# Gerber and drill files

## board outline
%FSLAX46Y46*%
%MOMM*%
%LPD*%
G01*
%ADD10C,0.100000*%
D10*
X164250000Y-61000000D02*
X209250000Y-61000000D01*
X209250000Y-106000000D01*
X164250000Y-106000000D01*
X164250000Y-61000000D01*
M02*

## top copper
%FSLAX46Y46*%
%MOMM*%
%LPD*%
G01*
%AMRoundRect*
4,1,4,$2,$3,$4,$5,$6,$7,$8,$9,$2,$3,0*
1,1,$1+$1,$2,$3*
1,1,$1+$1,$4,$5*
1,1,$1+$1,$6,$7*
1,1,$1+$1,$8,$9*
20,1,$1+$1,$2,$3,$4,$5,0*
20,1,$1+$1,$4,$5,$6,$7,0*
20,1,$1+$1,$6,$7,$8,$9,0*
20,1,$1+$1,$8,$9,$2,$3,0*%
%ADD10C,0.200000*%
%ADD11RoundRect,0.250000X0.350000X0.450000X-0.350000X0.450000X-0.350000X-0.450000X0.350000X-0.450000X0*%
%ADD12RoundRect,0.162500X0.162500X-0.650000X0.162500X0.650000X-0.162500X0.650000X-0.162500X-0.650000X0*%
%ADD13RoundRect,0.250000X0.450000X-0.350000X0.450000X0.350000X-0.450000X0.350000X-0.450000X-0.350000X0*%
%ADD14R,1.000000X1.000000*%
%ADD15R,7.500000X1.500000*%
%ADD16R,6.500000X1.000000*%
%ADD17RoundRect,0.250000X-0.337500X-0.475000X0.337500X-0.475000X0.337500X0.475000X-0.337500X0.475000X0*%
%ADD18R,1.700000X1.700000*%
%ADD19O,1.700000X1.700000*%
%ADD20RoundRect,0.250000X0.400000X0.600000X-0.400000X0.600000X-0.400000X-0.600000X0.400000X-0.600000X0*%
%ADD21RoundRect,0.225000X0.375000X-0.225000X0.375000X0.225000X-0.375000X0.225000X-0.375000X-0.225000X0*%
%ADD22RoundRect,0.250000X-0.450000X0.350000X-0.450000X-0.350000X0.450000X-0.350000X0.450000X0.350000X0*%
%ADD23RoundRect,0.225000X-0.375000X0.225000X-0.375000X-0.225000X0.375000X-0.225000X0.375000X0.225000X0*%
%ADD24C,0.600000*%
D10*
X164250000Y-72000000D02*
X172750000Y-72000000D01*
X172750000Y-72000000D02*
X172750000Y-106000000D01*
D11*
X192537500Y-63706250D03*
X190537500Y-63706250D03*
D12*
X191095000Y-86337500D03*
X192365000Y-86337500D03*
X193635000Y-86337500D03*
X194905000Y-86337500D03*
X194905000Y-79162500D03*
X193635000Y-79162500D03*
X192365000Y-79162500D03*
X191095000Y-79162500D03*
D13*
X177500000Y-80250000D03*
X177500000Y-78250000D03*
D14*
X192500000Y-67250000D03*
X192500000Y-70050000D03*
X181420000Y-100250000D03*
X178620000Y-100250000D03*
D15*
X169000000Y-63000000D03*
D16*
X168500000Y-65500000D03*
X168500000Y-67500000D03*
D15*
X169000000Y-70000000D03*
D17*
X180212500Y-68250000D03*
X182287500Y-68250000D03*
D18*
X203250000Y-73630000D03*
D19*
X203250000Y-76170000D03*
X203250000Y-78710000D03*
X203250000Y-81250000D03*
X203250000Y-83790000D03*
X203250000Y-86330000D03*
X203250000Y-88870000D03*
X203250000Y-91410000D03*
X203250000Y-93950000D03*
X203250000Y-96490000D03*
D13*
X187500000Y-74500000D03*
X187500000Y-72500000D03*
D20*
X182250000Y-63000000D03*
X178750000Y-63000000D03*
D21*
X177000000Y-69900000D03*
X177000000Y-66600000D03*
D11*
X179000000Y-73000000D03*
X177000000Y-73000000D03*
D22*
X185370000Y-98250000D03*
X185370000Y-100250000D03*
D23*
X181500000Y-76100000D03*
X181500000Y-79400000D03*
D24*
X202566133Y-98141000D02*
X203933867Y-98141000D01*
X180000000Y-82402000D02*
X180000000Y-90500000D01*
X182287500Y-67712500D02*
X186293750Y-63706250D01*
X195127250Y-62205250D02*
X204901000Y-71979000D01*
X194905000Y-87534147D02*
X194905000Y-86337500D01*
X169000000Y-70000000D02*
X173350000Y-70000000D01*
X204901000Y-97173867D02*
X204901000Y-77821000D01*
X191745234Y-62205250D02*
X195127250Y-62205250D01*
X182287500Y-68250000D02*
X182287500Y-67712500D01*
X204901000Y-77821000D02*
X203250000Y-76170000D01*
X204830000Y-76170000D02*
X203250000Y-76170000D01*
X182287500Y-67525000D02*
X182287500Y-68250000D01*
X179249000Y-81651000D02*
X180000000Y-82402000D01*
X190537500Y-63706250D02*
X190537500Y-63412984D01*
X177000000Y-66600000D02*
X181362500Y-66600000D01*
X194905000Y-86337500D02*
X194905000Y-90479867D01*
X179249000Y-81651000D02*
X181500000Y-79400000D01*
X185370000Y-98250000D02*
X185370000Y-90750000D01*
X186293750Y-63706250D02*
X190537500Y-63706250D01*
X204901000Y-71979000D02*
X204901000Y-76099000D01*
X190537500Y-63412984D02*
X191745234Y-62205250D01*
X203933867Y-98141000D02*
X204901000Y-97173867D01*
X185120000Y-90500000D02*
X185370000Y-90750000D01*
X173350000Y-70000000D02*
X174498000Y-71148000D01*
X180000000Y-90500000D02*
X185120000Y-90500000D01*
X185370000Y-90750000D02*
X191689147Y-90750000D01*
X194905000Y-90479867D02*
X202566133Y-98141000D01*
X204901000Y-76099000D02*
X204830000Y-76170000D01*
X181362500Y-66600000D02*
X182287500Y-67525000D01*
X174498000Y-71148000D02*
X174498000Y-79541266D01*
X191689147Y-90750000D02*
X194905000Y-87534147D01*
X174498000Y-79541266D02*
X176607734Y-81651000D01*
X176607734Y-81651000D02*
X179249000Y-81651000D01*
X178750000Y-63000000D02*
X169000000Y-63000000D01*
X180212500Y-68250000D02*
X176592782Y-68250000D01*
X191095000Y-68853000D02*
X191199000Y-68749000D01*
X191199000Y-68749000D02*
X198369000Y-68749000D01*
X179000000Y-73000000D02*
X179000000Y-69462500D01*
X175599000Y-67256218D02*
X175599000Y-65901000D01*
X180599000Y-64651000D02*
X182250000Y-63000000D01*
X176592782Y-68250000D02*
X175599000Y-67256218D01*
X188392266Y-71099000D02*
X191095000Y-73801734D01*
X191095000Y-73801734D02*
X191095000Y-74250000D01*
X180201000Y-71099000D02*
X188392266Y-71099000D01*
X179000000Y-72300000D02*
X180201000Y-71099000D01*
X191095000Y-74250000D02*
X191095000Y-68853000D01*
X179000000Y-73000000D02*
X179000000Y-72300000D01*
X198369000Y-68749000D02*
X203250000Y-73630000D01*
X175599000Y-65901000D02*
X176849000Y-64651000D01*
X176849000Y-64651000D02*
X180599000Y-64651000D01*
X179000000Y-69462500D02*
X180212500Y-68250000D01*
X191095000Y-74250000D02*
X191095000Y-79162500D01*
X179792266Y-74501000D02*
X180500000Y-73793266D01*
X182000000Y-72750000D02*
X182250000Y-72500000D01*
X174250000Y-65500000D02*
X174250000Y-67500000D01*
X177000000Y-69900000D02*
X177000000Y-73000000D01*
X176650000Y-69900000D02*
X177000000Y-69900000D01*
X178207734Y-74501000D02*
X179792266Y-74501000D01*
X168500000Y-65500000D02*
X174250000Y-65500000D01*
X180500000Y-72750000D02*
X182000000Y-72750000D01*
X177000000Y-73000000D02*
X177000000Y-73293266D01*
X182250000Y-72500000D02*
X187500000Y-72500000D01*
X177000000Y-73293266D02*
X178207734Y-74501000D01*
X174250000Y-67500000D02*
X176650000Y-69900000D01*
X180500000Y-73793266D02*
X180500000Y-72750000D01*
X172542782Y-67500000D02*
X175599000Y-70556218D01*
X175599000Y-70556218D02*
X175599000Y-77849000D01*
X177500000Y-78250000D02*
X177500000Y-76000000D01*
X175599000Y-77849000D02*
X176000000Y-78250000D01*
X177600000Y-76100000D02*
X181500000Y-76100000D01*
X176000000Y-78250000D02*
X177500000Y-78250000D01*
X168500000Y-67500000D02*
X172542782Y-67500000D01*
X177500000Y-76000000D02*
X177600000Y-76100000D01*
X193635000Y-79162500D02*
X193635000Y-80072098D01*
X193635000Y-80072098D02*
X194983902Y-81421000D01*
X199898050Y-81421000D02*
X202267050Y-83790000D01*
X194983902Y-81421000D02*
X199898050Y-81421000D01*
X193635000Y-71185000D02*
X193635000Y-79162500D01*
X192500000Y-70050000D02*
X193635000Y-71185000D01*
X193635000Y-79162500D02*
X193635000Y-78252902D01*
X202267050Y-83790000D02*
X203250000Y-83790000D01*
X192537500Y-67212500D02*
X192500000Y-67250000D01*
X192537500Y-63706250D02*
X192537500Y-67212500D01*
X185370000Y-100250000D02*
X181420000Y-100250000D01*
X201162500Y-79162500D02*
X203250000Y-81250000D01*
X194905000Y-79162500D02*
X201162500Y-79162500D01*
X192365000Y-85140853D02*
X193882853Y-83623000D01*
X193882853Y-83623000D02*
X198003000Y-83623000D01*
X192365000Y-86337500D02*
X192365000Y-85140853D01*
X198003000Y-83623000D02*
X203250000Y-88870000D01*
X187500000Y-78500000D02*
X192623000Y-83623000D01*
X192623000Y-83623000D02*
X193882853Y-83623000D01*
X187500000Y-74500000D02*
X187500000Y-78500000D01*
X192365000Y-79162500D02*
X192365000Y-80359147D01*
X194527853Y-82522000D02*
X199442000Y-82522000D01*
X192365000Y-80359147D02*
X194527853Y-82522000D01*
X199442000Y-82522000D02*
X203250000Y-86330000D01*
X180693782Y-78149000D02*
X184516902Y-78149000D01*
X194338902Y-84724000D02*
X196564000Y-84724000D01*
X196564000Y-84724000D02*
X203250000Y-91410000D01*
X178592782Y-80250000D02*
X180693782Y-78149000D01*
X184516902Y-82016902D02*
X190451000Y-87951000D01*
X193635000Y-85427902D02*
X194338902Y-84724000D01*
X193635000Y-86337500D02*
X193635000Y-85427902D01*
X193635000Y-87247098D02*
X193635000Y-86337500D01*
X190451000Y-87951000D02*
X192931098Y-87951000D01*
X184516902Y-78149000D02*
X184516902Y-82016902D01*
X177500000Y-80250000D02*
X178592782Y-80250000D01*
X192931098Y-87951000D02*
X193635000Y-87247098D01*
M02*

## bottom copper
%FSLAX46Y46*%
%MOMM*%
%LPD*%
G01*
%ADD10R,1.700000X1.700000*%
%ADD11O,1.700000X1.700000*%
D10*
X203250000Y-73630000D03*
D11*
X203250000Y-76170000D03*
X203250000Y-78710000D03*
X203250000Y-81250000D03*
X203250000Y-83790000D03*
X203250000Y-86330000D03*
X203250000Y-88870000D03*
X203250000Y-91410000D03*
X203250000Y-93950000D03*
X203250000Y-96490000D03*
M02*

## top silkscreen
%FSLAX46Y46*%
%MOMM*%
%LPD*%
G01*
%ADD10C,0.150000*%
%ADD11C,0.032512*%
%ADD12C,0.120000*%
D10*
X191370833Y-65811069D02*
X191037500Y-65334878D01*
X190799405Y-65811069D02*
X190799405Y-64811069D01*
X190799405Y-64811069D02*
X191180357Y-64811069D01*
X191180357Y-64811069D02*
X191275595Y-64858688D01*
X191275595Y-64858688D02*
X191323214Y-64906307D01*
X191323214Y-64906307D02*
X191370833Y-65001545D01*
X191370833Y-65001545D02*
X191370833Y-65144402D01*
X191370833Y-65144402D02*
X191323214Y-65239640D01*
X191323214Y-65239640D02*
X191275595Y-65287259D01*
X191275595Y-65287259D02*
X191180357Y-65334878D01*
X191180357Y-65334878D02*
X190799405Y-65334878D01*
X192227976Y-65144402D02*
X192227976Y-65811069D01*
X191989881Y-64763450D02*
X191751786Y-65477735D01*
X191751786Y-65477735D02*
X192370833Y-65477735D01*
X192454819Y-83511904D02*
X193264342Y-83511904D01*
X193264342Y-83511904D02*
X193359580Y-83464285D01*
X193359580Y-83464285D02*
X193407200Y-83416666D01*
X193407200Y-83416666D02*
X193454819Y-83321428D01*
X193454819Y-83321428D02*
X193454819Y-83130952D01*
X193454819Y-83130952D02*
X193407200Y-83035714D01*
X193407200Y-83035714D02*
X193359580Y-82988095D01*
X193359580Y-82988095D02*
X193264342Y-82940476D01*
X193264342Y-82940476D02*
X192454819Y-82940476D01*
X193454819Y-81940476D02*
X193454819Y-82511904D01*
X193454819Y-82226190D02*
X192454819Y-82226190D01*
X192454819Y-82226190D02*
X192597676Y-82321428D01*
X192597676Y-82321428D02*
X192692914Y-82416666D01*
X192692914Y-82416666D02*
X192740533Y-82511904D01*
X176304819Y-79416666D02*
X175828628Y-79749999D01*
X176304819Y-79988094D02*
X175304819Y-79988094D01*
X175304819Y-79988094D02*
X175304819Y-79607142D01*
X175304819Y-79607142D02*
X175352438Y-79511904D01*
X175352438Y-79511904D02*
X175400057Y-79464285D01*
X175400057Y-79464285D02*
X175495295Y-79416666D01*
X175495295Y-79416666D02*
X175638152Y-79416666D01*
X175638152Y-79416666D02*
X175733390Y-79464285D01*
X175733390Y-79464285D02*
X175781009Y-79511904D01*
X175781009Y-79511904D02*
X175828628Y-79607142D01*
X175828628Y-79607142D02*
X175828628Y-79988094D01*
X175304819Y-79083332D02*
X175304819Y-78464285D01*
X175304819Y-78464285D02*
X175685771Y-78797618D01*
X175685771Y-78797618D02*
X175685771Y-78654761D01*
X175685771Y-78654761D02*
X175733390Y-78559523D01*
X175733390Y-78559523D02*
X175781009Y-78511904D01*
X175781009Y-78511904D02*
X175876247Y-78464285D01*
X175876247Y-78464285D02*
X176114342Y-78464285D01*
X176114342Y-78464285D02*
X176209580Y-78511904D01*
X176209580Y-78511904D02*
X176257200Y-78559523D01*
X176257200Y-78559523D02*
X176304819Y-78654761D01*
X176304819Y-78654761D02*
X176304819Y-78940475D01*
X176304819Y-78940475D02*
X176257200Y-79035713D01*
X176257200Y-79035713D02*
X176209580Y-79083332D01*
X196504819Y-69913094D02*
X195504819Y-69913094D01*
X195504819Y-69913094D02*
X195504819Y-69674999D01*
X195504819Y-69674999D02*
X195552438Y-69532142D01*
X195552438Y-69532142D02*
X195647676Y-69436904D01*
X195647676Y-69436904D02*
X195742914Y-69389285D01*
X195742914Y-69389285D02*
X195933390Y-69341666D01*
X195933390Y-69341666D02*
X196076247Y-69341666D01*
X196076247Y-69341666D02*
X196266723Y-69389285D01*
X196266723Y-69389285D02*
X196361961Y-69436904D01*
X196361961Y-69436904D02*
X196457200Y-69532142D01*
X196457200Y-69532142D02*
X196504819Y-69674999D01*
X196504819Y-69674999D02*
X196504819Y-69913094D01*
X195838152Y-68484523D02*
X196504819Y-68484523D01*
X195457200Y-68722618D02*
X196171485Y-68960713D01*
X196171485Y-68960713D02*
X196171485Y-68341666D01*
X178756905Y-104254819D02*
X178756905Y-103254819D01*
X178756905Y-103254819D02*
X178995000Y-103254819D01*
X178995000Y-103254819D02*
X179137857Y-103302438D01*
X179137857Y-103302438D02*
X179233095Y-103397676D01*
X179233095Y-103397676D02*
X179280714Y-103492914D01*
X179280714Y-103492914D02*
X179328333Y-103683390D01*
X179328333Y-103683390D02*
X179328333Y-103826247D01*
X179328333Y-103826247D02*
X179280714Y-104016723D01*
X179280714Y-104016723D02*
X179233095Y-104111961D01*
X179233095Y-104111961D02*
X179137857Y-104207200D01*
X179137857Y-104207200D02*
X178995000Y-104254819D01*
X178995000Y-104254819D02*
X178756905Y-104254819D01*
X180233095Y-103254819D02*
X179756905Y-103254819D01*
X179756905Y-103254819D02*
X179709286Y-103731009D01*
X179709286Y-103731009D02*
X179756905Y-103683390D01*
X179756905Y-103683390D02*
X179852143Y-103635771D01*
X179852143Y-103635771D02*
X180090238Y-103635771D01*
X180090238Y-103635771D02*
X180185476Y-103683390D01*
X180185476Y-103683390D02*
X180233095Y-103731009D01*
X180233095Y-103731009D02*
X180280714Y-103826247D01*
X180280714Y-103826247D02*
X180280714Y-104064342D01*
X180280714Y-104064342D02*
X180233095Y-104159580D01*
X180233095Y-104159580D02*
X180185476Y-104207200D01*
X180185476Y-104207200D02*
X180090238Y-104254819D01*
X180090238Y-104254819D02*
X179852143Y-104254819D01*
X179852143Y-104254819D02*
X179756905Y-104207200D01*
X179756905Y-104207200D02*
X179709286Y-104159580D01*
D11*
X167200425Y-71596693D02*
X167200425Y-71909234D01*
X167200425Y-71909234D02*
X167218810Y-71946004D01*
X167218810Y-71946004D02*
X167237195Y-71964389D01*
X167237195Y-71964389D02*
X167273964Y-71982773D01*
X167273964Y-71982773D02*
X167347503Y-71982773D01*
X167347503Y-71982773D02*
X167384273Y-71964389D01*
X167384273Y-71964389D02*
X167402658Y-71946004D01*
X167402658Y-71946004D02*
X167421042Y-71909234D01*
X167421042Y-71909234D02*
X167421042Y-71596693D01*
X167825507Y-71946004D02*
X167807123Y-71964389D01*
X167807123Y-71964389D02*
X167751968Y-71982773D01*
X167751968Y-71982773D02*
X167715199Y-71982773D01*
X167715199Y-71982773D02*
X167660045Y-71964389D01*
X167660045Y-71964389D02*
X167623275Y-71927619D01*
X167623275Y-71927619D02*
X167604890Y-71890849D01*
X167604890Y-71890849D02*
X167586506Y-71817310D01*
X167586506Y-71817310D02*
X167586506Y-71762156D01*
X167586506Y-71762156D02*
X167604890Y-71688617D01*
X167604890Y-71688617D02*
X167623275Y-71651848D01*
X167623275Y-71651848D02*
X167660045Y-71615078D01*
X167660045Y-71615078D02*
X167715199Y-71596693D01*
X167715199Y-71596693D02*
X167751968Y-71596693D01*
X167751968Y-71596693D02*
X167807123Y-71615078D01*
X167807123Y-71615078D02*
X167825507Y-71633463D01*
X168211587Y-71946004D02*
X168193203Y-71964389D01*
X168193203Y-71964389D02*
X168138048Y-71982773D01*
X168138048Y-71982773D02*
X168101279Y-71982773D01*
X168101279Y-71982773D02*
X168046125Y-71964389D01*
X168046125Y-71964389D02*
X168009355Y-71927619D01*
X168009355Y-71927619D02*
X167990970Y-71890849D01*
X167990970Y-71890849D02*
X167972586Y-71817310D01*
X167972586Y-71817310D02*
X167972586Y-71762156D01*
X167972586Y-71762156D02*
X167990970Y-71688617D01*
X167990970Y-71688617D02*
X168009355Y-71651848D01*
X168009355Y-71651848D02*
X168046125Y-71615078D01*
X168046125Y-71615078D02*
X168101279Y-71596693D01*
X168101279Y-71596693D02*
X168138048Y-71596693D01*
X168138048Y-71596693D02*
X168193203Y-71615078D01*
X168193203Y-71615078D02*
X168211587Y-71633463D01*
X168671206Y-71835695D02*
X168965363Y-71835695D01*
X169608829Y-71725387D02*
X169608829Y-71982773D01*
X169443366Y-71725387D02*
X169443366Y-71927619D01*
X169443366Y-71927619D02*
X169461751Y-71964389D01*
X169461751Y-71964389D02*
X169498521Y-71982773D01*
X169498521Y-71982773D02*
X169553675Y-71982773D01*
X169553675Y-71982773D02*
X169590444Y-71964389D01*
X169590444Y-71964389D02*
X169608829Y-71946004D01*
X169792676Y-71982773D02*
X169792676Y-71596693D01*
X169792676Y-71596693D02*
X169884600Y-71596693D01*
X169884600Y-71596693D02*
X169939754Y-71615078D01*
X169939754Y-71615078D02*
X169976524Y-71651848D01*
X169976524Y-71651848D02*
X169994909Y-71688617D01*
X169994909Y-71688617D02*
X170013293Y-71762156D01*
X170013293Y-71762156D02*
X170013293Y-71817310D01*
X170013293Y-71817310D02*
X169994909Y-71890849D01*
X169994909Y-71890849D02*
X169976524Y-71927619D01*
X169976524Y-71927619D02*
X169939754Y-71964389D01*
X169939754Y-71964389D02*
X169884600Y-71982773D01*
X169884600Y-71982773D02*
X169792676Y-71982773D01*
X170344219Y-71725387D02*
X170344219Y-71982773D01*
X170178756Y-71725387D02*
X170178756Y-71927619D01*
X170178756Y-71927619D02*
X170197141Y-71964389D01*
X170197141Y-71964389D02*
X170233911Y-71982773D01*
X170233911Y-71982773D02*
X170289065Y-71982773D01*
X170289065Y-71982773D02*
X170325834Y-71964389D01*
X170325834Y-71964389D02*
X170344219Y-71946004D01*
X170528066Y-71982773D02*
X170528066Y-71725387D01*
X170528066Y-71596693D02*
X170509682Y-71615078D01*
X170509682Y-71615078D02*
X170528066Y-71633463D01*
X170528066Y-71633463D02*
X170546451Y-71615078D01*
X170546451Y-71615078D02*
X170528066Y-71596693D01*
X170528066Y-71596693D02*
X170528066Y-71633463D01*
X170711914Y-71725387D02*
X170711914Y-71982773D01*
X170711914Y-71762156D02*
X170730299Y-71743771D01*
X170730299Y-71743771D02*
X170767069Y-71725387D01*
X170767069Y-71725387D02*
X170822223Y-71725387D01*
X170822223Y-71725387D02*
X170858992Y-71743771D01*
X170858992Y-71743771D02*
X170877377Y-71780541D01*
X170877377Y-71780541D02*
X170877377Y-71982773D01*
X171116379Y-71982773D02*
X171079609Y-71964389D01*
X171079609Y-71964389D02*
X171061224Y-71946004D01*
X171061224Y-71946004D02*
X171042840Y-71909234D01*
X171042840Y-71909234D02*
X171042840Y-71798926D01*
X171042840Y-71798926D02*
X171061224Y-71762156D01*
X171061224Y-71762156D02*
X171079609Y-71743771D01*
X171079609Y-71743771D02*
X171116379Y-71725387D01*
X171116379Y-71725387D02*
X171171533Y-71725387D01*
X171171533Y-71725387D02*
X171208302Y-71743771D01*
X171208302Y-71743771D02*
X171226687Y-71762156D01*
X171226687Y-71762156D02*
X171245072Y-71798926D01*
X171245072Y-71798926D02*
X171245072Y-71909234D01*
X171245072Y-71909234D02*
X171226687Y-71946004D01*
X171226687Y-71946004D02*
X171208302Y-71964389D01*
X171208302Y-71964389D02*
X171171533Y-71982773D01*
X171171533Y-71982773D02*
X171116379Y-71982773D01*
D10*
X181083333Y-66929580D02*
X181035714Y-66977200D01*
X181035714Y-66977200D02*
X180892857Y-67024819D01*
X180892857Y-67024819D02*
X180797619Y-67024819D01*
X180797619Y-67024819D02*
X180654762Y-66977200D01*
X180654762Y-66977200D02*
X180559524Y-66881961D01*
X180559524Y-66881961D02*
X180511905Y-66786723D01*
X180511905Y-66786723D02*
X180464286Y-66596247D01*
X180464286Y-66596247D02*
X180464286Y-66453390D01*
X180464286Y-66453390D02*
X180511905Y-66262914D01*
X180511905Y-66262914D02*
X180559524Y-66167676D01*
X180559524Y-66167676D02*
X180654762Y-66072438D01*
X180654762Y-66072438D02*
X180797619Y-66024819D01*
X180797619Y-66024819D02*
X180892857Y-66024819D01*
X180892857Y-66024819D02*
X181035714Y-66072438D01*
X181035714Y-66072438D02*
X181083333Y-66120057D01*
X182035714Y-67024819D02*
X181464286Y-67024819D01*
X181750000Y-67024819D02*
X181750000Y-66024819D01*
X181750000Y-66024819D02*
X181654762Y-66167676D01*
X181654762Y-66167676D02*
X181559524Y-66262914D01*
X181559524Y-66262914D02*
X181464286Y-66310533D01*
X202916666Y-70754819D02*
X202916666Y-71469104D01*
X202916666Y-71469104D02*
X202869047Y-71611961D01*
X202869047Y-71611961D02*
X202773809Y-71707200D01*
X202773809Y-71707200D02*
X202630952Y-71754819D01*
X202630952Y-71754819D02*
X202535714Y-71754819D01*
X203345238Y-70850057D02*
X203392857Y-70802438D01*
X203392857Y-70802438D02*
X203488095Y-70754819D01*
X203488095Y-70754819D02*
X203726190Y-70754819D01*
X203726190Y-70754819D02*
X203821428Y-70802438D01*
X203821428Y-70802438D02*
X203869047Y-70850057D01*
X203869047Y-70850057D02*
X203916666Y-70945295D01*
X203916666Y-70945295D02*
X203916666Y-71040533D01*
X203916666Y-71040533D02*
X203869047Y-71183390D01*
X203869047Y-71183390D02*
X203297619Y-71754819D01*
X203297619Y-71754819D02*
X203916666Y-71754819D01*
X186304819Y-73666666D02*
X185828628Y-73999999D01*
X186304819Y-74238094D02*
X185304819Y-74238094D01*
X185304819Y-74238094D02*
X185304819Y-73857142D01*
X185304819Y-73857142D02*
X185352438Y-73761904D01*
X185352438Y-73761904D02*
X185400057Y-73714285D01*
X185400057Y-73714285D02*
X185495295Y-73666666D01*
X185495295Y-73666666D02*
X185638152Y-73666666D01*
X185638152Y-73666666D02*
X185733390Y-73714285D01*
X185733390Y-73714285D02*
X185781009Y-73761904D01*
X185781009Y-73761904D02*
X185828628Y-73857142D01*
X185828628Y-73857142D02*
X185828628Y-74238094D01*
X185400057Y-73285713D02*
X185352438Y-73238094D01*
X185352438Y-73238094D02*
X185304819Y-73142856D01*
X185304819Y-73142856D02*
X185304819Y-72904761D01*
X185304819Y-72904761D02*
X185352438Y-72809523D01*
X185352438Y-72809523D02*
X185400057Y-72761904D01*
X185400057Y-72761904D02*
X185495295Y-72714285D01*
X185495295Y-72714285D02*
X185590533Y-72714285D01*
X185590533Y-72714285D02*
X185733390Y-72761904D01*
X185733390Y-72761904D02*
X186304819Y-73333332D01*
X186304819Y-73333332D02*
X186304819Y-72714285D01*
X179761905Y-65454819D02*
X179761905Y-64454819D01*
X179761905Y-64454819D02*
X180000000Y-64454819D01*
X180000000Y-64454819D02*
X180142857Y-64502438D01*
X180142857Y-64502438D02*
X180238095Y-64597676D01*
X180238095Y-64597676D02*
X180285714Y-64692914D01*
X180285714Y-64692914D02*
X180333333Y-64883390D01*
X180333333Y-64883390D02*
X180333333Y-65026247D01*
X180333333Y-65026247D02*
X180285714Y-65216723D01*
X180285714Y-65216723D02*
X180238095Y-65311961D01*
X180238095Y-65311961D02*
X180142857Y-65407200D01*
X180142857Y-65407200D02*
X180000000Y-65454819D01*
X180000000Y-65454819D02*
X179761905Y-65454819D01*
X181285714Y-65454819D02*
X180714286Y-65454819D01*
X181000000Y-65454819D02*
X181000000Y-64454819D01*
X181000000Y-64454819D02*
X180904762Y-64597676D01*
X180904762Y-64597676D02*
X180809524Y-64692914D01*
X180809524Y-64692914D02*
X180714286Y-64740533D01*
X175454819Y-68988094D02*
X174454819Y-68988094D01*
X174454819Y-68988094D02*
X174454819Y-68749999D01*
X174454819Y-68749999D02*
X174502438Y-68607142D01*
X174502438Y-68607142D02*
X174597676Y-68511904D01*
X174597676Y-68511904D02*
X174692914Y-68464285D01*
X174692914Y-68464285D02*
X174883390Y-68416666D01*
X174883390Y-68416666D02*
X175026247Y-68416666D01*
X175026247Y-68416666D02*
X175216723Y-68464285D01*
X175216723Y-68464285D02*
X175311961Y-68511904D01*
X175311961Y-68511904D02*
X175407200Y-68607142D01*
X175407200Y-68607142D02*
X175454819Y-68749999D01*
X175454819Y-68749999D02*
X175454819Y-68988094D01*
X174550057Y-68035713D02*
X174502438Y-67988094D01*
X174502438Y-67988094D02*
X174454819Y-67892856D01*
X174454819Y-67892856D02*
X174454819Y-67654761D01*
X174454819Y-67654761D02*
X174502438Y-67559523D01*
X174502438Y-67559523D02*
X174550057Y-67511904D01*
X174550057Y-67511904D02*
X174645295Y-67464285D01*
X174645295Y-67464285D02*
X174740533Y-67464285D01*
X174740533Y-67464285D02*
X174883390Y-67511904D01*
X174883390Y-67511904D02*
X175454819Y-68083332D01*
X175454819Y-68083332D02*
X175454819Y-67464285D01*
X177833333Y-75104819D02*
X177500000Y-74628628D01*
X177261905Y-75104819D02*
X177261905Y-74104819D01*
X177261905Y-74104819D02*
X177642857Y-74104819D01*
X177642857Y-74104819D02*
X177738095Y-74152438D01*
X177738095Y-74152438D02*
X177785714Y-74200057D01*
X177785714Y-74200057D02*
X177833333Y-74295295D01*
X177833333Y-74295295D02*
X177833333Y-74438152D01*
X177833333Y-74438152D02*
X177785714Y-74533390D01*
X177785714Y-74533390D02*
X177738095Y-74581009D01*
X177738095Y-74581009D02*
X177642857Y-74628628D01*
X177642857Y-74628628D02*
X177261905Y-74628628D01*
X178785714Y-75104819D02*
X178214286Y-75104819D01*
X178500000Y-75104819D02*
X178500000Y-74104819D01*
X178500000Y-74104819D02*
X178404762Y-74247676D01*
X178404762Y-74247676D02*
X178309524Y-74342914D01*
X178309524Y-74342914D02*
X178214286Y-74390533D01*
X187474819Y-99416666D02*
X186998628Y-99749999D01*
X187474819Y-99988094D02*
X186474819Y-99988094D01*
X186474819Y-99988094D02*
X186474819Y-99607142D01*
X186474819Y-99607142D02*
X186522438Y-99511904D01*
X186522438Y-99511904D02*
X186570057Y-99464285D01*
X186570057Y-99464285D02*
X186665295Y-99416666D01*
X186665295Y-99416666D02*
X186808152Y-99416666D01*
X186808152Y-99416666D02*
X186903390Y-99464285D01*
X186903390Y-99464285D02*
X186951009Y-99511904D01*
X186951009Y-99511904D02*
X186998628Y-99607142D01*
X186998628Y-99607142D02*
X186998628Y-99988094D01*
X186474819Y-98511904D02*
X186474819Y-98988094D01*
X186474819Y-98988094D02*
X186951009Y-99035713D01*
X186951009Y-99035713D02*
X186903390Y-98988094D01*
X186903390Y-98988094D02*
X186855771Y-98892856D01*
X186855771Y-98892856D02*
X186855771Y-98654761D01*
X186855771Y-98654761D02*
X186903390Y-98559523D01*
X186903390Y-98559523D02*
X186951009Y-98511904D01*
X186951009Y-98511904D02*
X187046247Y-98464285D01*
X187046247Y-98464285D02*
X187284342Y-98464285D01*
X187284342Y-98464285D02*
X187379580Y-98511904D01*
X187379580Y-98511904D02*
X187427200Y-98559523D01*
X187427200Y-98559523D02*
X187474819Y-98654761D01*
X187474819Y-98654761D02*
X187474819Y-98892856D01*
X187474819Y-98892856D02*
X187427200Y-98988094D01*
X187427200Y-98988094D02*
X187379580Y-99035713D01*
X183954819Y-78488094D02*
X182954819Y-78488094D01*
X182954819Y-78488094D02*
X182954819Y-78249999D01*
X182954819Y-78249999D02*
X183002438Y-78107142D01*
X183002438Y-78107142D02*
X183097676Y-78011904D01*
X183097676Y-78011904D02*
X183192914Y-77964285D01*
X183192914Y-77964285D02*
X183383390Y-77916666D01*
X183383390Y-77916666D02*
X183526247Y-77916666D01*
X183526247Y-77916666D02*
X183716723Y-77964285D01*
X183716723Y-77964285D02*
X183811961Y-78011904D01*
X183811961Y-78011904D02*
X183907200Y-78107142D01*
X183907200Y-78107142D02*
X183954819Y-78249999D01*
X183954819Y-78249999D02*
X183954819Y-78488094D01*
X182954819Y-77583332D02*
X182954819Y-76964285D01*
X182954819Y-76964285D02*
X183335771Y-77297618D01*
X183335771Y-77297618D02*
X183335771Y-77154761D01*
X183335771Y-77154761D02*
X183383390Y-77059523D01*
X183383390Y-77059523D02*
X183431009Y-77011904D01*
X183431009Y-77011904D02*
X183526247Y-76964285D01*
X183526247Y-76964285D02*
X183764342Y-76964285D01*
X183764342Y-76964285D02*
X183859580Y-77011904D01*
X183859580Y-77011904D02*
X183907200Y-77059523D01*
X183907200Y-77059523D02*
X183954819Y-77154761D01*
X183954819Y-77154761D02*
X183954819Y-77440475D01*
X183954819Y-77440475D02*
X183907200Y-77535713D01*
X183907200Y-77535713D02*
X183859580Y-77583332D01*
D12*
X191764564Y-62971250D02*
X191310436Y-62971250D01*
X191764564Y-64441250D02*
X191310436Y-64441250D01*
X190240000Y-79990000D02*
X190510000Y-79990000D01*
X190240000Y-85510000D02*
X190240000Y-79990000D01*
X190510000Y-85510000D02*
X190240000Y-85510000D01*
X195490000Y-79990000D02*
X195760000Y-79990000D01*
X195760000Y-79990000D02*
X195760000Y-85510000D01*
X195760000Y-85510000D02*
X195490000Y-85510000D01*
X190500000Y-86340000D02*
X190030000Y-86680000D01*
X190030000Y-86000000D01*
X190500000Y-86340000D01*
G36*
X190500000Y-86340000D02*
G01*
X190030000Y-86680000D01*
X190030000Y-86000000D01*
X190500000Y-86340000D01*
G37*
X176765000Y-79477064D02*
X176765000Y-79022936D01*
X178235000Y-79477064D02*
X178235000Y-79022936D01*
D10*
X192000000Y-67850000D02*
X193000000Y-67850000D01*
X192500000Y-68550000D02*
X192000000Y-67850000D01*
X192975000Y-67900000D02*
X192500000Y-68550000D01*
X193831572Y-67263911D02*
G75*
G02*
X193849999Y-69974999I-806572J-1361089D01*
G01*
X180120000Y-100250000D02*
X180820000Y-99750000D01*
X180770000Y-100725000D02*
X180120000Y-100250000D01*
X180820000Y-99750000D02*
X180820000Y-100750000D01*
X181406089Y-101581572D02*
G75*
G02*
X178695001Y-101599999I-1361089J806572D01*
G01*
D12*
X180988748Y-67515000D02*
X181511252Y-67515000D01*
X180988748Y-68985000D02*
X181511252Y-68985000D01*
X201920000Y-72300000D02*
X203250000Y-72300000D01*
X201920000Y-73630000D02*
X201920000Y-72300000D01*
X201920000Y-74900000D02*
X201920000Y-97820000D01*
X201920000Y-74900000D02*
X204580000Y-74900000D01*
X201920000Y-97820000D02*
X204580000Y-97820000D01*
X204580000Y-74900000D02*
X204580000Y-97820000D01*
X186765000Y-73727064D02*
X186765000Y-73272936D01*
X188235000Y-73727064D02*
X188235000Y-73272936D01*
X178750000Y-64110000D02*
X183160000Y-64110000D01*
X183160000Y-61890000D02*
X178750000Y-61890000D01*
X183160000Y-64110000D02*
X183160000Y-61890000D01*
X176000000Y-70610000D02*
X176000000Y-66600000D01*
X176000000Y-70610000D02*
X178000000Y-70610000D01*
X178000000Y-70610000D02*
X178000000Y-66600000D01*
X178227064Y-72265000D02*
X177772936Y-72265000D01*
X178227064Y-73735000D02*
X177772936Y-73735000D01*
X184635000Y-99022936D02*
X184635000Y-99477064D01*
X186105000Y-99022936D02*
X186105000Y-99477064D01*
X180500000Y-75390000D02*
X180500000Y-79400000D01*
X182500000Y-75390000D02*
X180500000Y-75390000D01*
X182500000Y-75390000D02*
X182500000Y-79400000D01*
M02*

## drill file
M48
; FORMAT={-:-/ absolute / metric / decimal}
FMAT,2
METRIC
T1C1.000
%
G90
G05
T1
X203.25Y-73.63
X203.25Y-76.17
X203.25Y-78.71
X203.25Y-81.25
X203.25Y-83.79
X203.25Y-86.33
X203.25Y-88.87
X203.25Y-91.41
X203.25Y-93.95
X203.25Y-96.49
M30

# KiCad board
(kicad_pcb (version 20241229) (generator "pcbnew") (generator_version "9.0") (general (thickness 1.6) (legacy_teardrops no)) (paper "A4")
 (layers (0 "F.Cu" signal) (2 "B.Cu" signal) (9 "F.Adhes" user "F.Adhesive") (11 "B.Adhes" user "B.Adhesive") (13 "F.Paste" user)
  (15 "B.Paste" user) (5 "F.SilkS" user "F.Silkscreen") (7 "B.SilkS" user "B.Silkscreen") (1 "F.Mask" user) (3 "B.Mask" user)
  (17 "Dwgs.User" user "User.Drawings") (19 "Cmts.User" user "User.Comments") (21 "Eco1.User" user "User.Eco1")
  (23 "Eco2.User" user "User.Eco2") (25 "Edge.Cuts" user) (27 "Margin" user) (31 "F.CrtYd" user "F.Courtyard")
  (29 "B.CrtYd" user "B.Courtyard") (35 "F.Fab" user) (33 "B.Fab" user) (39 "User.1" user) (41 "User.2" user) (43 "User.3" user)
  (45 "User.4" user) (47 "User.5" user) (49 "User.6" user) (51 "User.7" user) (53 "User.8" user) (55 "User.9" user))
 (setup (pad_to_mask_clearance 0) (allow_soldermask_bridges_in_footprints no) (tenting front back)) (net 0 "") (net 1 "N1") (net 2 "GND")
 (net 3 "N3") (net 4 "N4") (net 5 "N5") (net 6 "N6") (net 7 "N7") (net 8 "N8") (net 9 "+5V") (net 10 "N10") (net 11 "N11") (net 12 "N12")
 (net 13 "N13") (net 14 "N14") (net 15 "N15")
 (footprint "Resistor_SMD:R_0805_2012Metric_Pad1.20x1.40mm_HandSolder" (layer "F.Cu") (at 191.5375 63.70625 180)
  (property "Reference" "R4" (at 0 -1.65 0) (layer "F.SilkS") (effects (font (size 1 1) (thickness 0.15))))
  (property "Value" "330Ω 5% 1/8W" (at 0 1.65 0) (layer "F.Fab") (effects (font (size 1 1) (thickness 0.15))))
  (fp_line (start -0.227064 0.735) (end 0.227064 0.735) (stroke (width 0.12) (type solid)) (layer "F.SilkS"))
  (fp_line (start -0.227064 -0.735) (end 0.227064 -0.735) (stroke (width 0.12) (type solid)) (layer "F.SilkS"))
  (pad "1" smd roundrect (at -1 0 180) (size 1.2 1.4) (layers "F.Cu" "F.Mask" "F.Paste") (roundrect_rratio 0.208333) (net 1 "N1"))
  (pad "2" smd roundrect (at 1 0 180) (size 1.2 1.4) (layers "F.Cu" "F.Mask" "F.Paste") (roundrect_rratio 0.208333) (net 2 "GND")))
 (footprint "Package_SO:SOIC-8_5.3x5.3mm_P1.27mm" (layer "F.Cu") (at 193 82.75 90)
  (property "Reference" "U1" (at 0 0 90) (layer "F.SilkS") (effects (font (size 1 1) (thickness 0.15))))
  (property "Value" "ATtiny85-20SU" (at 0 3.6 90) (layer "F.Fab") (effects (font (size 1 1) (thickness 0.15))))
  (fp_line (start 2.76 -2.76) (end 2.76 -2.49) (stroke (width 0.12) (type solid)) (layer "F.SilkS"))
  (fp_line (start -2.76 -2.76) (end 2.76 -2.76) (stroke (width 0.12) (type solid)) (layer "F.SilkS"))
  (fp_line (start -2.76 -2.49) (end -2.76 -2.76) (stroke (width 0.12) (type solid)) (layer "F.SilkS"))
  (fp_line (start 2.76 2.49) (end 2.76 2.76) (stroke (width 0.12) (type solid)) (layer "F.SilkS"))
  (fp_line (start 2.76 2.76) (end -2.76 2.76) (stroke (width 0.12) (type solid)) (layer "F.SilkS"))
  (fp_line (start -2.76 2.76) (end -2.76 2.49) (stroke (width 0.12) (type solid)) (layer "F.SilkS"))
  (fp_poly (pts (xy -3.59 -2.5) (xy -3.93 -2.97) (xy -3.25 -2.97)) (stroke (width 0.12) (type solid)) (fill yes) (layer "F.SilkS"))
  (pad "1" smd roundrect (at -3.5875 -1.905 90) (size 1.625 0.65) (layers "F.Cu" "F.Mask" "F.Paste") (roundrect_rratio 0.25) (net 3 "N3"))
  (pad "2" smd roundrect (at -3.5875 -0.635 90) (size 1.625 0.65) (layers "F.Cu" "F.Mask" "F.Paste") (roundrect_rratio 0.25) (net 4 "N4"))
  (pad "3" smd roundrect (at -3.5875 0.635 90) (size 1.625 0.65) (layers "F.Cu" "F.Mask" "F.Paste") (roundrect_rratio 0.25) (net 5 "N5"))
  (pad "4" smd roundrect (at -3.5875 1.905 90) (size 1.625 0.65) (layers "F.Cu" "F.Mask" "F.Paste") (roundrect_rratio 0.25) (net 2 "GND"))
  (pad "5" smd roundrect (at 3.5875 1.905 90) (size 1.625 0.65) (layers "F.Cu" "F.Mask" "F.Paste") (roundrect_rratio 0.25) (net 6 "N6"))
  (pad "6" smd roundrect (at 3.5875 0.635 90) (size 1.625 0.65) (layers "F.Cu" "F.Mask" "F.Paste") (roundrect_rratio 0.25) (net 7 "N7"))
  (pad "7" smd roundrect (at 3.5875 -0.635 90) (size 1.625 0.65) (layers "F.Cu" "F.Mask" "F.Paste") (roundrect_rratio 0.25) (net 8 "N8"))
  (pad "8" smd roundrect (at 3.5875 -1.905 90) (size 1.625 0.65) (layers "F.Cu" "F.Mask" "F.Paste") (roundrect_rratio 0.25) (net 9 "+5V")))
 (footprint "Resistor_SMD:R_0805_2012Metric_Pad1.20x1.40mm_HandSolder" (layer "F.Cu") (at 177.5 79.25 90)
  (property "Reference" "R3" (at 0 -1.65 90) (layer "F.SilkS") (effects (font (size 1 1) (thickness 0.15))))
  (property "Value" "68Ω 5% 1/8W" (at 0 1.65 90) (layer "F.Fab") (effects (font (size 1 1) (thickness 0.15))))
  (fp_line (start -0.227064 -0.735) (end 0.227064 -0.735) (stroke (width 0.12) (type solid)) (layer "F.SilkS"))
  (fp_line (start -0.227064 0.735) (end 0.227064 0.735) (stroke (width 0.12) (type solid)) (layer "F.SilkS"))
  (pad "1" smd roundrect (at -1 0 90) (size 1.2 1.4) (layers "F.Cu" "F.Mask" "F.Paste") (roundrect_rratio 0.208333) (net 5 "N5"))
  (pad "2" smd roundrect (at 1 0 90) (size 1.2 1.4) (layers "F.Cu" "F.Mask" "F.Paste") (roundrect_rratio 0.208333) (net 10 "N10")))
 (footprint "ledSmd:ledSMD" (layer "F.Cu") (at 192.5 69.05 -90)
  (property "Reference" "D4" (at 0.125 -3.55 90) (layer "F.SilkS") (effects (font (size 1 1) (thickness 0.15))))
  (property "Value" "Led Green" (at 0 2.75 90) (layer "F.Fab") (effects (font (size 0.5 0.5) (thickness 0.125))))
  (fp_line (start -1.2 0.5) (end -1.2 -0.5) (stroke (width 0.15) (type solid)) (layer "F.SilkS"))
  (fp_line (start -0.5 0) (end -1.2 0.5) (stroke (width 0.15) (type solid)) (layer "F.SilkS"))
  (fp_line (start -1.15 -0.475) (end -0.5 0) (stroke (width 0.15) (type solid)) (layer "F.SilkS"))
  (fp_arc (start -1.786089 -1.331572) (mid -0.435753 -2.107089) (end 0.924999 -1.349999) (stroke (width 0.15) (type solid))
   (layer "F.SilkS"))
  (pad "1" smd rect (at -1.8 0 270) (size 1 1) (layers "F.Cu" "F.Mask" "F.Paste") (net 1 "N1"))
  (pad "2" smd rect (at 1 0 270) (size 1 1) (layers "F.Cu" "F.Mask" "F.Paste") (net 7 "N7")))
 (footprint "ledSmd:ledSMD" (layer "F.Cu") (at 179.62 100.25 180)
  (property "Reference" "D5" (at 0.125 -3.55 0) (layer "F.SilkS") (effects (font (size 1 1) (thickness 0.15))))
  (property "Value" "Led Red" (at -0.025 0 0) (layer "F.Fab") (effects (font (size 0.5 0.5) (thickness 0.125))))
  (fp_line (start -0.5 0) (end -1.2 0.5) (stroke (width 0.15) (type solid)) (layer "F.SilkS"))
  (fp_line (start -1.15 -0.475) (end -0.5 0) (stroke (width 0.15) (type solid)) (layer "F.SilkS"))
  (fp_line (start -1.2 0.5) (end -1.2 -0.5) (stroke (width 0.15) (type solid)) (layer "F.SilkS"))
  (fp_arc (start -1.786089 -1.331572) (mid -0.435753 -2.107089) (end 0.924999 -1.349999) (stroke (width 0.15) (type solid))
   (layer "F.SilkS"))
  (pad "1" smd rect (at -1.8 0 180) (size 1 1) (layers "F.Cu" "F.Mask" "F.Paste") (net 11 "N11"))
  (pad "2" smd rect (at 1 0 180) (size 1 1) (layers "F.Cu" "F.Mask" "F.Paste") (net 9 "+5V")))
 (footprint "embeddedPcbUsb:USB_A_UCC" (layer "F.Cu") (at 168.8 66.5 180)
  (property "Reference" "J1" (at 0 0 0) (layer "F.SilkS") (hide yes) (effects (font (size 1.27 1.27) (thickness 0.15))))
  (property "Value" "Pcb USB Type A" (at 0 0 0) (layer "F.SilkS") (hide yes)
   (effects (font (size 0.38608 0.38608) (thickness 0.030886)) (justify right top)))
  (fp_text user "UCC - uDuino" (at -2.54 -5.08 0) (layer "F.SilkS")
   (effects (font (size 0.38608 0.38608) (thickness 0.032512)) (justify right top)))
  (pad "1" smd rect (at -0.2 3.5 180) (size 7.5 1.5) (layers "F.Cu" "F.Mask" "F.Paste") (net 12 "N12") (solder_mask_margin 0.1016))
  (pad "2" smd rect (at 0.3 1 180) (size 6.5 1) (layers "F.Cu" "F.Mask" "F.Paste") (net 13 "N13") (solder_mask_margin 0.1016))
  (pad "3" smd rect (at 0.3 -1 180) (size 6.5 1) (layers "F.Cu" "F.Mask" "F.Paste") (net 10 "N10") (solder_mask_margin 0.1016))
  (pad "4" smd rect (at -0.2 -3.5 180) (size 7.5 1.5) (layers "F.Cu" "F.Mask" "F.Paste") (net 2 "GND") (solder_mask_margin 0.1016)))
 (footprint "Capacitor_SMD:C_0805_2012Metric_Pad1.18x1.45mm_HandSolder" (layer "F.Cu") (at 181.25 68.25)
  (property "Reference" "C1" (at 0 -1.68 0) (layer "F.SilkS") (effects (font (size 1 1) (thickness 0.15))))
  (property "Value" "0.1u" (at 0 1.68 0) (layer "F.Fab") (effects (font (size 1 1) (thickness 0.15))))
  (fp_line (start -0.261252 -0.735) (end 0.261252 -0.735) (stroke (width 0.12) (type solid)) (layer "F.SilkS"))
  (fp_line (start -0.261252 0.735) (end 0.261252 0.735) (stroke (width 0.12) (type solid)) (layer "F.SilkS"))
  (pad "1" smd roundrect (at -1.0375 0) (size 1.175 1.45) (layers "F.Cu" "F.Mask" "F.Paste") (roundrect_rratio 0.212766) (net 9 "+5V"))
  (pad "2" smd roundrect (at 1.0375 0) (size 1.175 1.45) (layers "F.Cu" "F.Mask" "F.Paste") (roundrect_rratio 0.212766) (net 2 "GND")))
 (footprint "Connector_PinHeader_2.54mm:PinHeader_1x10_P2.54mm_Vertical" (layer "F.Cu") (at 203.25 73.63)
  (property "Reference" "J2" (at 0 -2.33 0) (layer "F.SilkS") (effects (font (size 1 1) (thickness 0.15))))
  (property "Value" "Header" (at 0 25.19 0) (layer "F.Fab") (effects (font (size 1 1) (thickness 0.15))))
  (fp_line (start -1.33 -1.33) (end 0 -1.33) (stroke (width 0.12) (type solid)) (layer "F.SilkS"))
  (fp_line (start -1.33 0) (end -1.33 -1.33) (stroke (width 0.12) (type solid)) (layer "F.SilkS"))
  (fp_line (start -1.33 1.27) (end -1.33 24.19) (stroke (width 0.12) (type solid)) (layer "F.SilkS"))
  (fp_line (start -1.33 1.27) (end 1.33 1.27) (stroke (width 0.12) (type solid)) (layer "F.SilkS"))
  (fp_line (start -1.33 24.19) (end 1.33 24.19) (stroke (width 0.12) (type solid)) (layer "F.SilkS"))
  (fp_line (start 1.33 1.27) (end 1.33 24.19) (stroke (width 0.12) (type solid)) (layer "F.SilkS"))
  (pad "1" thru_hole rect (at 0 0) (size 1.7 1.7) (drill 1) (layers "*.Cu" "*.Mask") (remove_unused_layers no) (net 9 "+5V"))
  (pad "2" thru_hole oval (at 0 2.54) (size 1.7 1.7) (drill 1) (layers "*.Cu" "*.Mask") (remove_unused_layers no) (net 2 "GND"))
  (pad "3" thru_hole oval (at 0 5.08) (size 1.7 1.7) (drill 1) (layers "*.Cu" "*.Mask") (remove_unused_layers no) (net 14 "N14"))
  (pad "4" thru_hole oval (at 0 7.62) (size 1.7 1.7) (drill 1) (layers "*.Cu" "*.Mask") (remove_unused_layers no) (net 6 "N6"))
  (pad "5" thru_hole oval (at 0 10.16) (size 1.7 1.7) (drill 1) (layers "*.Cu" "*.Mask") (remove_unused_layers no) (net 7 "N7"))
  (pad "6" thru_hole oval (at 0 12.7) (size 1.7 1.7) (drill 1) (layers "*.Cu" "*.Mask") (remove_unused_layers no) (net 8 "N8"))
  (pad "7" thru_hole oval (at 0 15.24) (size 1.7 1.7) (drill 1) (layers "*.Cu" "*.Mask") (remove_unused_layers no) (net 4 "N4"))
  (pad "8" thru_hole oval (at 0 17.78) (size 1.7 1.7) (drill 1) (layers "*.Cu" "*.Mask") (remove_unused_layers no) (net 5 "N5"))
  (pad "9" thru_hole oval (at 0 20.32) (size 1.7 1.7) (drill 1) (layers "*.Cu" "*.Mask") (remove_unused_layers no) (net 3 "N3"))
  (pad "10" thru_hole oval (at 0 22.86) (size 1.7 1.7) (drill 1) (layers "*.Cu" "*.Mask") (remove_unused_layers no) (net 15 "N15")))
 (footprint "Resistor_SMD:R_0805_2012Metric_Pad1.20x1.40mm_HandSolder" (layer "F.Cu") (at 187.5 73.5 90)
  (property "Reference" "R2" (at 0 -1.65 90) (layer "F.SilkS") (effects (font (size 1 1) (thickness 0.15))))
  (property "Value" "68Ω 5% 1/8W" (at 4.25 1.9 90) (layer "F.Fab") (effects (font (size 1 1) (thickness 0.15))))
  (fp_line (start -0.227064 -0.735) (end 0.227064 -0.735) (stroke (width 0.12) (type solid)) (layer "F.SilkS"))
  (fp_line (start -0.227064 0.735) (end 0.227064 0.735) (stroke (width 0.12) (type solid)) (layer "F.SilkS"))
  (pad "1" smd roundrect (at -1 0 90) (size 1.2 1.4) (layers "F.Cu" "F.Mask" "F.Paste") (roundrect_rratio 0.208333) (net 4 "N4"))
  (pad "2" smd roundrect (at 1 0 90) (size 1.2 1.4) (layers "F.Cu" "F.Mask" "F.Paste") (roundrect_rratio 0.208333) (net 13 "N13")))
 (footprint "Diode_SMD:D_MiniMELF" (layer "F.Cu") (at 180.5 63 180)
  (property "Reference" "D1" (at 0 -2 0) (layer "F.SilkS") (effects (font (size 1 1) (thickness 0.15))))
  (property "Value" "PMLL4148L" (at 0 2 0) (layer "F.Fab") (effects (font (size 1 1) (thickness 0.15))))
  (fp_line (start 1.75 -1.11) (end -2.66 -1.11) (stroke (width 0.12) (type solid)) (layer "F.SilkS"))
  (fp_line (start -2.66 1.11) (end 1.75 1.11) (stroke (width 0.12) (type solid)) (layer "F.SilkS"))
  (fp_line (start -2.66 -1.11) (end -2.66 1.11) (stroke (width 0.12) (type solid)) (layer "F.SilkS"))
  (pad "1" smd roundrect (at -1.75 0 180) (size 1.3 1.7) (layers "F.Cu" "F.Mask" "F.Paste") (roundrect_rratio 0.1923076923) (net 9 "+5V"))
  (pad "2" smd roundrect (at 1.75 0 180) (size 1.3 1.7) (layers "F.Cu" "F.Mask" "F.Paste") (roundrect_rratio 0.1923076923) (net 12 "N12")))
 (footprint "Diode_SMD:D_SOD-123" (layer "F.Cu") (at 177 68.25 90)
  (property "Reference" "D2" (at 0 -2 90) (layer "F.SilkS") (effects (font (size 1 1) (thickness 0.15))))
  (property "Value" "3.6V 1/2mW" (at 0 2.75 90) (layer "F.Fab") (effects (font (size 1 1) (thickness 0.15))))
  (fp_line (start -2.36 -1) (end 1.65 -1) (stroke (width 0.12) (type solid)) (layer "F.SilkS"))
  (fp_line (start -2.36 -1) (end -2.36 1) (stroke (width 0.12) (type solid)) (layer "F.SilkS"))
  (fp_line (start -2.36 1) (end 1.65 1) (stroke (width 0.12) (type solid)) (layer "F.SilkS"))
  (pad "1" smd roundrect (at -1.65 0 90) (size 0.9 1.2) (layers "F.Cu" "F.Mask" "F.Paste") (roundrect_rratio 0.25) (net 13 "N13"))
  (pad "2" smd roundrect (at 1.65 0 90) (size 0.9 1.2) (layers "F.Cu" "F.Mask" "F.Paste") (roundrect_rratio 0.25) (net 2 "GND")))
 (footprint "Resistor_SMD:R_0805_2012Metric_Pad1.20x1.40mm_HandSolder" (layer "F.Cu") (at 178 73 180)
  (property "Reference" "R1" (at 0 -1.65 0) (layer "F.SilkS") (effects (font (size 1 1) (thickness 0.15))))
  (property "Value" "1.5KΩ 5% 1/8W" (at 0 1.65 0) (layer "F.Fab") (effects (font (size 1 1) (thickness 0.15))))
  (fp_line (start -0.227064 0.735) (end 0.227064 0.735) (stroke (width 0.12) (type solid)) (layer "F.SilkS"))
  (fp_line (start -0.227064 -0.735) (end 0.227064 -0.735) (stroke (width 0.12) (type solid)) (layer "F.SilkS"))
  (pad "1" smd roundrect (at -1 0 180) (size 1.2 1.4) (layers "F.Cu" "F.Mask" "F.Paste") (roundrect_rratio 0.208333) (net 9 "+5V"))
  (pad "2" smd roundrect (at 1 0 180) (size 1.2 1.4) (layers "F.Cu" "F.Mask" "F.Paste") (roundrect_rratio 0.208333) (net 13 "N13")))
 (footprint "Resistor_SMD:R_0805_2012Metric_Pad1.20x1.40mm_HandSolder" (layer "F.Cu") (at 185.37 99.25 -90)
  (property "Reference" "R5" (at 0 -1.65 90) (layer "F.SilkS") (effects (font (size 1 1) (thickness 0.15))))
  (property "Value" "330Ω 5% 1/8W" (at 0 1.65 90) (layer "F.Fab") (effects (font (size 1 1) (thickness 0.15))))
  (fp_line (start -0.227064 0.735) (end 0.227064 0.735) (stroke (width 0.12) (type solid)) (layer "F.SilkS"))
  (fp_line (start -0.227064 -0.735) (end 0.227064 -0.735) (stroke (width 0.12) (type solid)) (layer "F.SilkS"))
  (pad "1" smd roundrect (at -1 0 270) (size 1.2 1.4) (layers "F.Cu" "F.Mask" "F.Paste") (roundrect_rratio 0.208333) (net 2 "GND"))
  (pad "2" smd roundrect (at 1 0 270) (size 1.2 1.4) (layers "F.Cu" "F.Mask" "F.Paste") (roundrect_rratio 0.208333) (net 11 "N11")))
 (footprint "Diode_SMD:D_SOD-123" (layer "F.Cu") (at 181.5 77.75 -90)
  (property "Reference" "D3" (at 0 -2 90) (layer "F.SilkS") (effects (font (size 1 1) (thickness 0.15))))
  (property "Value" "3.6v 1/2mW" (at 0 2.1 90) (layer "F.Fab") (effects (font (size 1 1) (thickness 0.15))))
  (fp_line (start -2.36 1) (end 1.65 1) (stroke (width 0.12) (type solid)) (layer "F.SilkS"))
  (fp_line (start -2.36 -1) (end -2.36 1) (stroke (width 0.12) (type solid)) (layer "F.SilkS"))
  (fp_line (start -2.36 -1) (end 1.65 -1) (stroke (width 0.12) (type solid)) (layer "F.SilkS"))
  (pad "1" smd roundrect (at -1.65 0 270) (size 0.9 1.2) (layers "F.Cu" "F.Mask" "F.Paste") (roundrect_rratio 0.25) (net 10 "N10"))
  (pad "2" smd roundrect (at 1.65 0 270) (size 0.9 1.2) (layers "F.Cu" "F.Mask" "F.Paste") (roundrect_rratio 0.25) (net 2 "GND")))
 (gr_line (start 164.25 72) (end 172.75 72) (stroke (width 0.2) (type default)) (layer "F.Cu"))
 (gr_line (start 172.75 72) (end 172.75 106) (stroke (width 0.2) (type default)) (layer "F.Cu"))
 (gr_rect (start 164.25 61) (end 209.25 106) (stroke (width 0.1) (type default)) (fill no) (layer "Edge.Cuts"))
 (segment (start 202.566133 98.141) (end 203.933867 98.141) (width 0.6) (layer "F.Cu") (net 2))
 (segment (start 180 82.402) (end 180 90.5) (width 0.6) (layer "F.Cu") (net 2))
 (segment (start 182.2875 67.7125) (end 186.29375 63.70625) (width 0.6) (layer "F.Cu") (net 2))
 (segment (start 195.12725 62.20525) (end 204.901 71.979) (width 0.6) (layer "F.Cu") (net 2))
 (segment (start 194.905 87.534147) (end 194.905 86.3375) (width 0.6) (layer "F.Cu") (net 2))
 (segment (start 169 70) (end 173.35 70) (width 0.6) (layer "F.Cu") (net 2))
 (segment (start 204.901 97.173867) (end 204.901 77.821) (width 0.6) (layer "F.Cu") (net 2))
 (segment (start 191.745234 62.20525) (end 195.12725 62.20525) (width 0.6) (layer "F.Cu") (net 2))
 (segment (start 182.2875 68.25) (end 182.2875 67.7125) (width 0.6) (layer "F.Cu") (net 2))
 (segment (start 204.901 77.821) (end 203.25 76.17) (width 0.6) (layer "F.Cu") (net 2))
 (segment (start 204.83 76.17) (end 203.25 76.17) (width 0.6) (layer "F.Cu") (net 2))
 (segment (start 182.2875 67.525) (end 182.2875 68.25) (width 0.6) (layer "F.Cu") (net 2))
 (segment (start 179.249 81.651) (end 180 82.402) (width 0.6) (layer "F.Cu") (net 2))
 (segment (start 190.5375 63.70625) (end 190.5375 63.412984) (width 0.6) (layer "F.Cu") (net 2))
 (segment (start 177 66.6) (end 181.3625 66.6) (width 0.6) (layer "F.Cu") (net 2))
 (segment (start 194.905 86.3375) (end 194.905 90.479867) (width 0.6) (layer "F.Cu") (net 2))
 (segment (start 179.249 81.651) (end 181.5 79.4) (width 0.6) (layer "F.Cu") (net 2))
 (segment (start 185.37 98.25) (end 185.37 90.75) (width 0.6) (layer "F.Cu") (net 2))
 (segment (start 186.29375 63.70625) (end 190.5375 63.70625) (width 0.6) (layer "F.Cu") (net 2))
 (segment (start 204.901 71.979) (end 204.901 76.099) (width 0.6) (layer "F.Cu") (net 2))
 (segment (start 190.5375 63.412984) (end 191.745234 62.20525) (width 0.6) (layer "F.Cu") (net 2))
 (segment (start 203.933867 98.141) (end 204.901 97.173867) (width 0.6) (layer "F.Cu") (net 2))
 (segment (start 185.12 90.5) (end 185.37 90.75) (width 0.6) (layer "F.Cu") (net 2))
 (segment (start 173.35 70) (end 174.498 71.148) (width 0.6) (layer "F.Cu") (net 2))
 (segment (start 180 90.5) (end 185.12 90.5) (width 0.6) (layer "F.Cu") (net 2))
 (segment (start 185.37 90.75) (end 191.689147 90.75) (width 0.6) (layer "F.Cu") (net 2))
 (segment (start 194.905 90.479867) (end 202.566133 98.141) (width 0.6) (layer "F.Cu") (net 2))
 (segment (start 204.901 76.099) (end 204.83 76.17) (width 0.6) (layer "F.Cu") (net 2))
 (segment (start 181.3625 66.6) (end 182.2875 67.525) (width 0.6) (layer "F.Cu") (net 2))
 (segment (start 174.498 71.148) (end 174.498 79.541266) (width 0.6) (layer "F.Cu") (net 2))
 (segment (start 191.689147 90.75) (end 194.905 87.534147) (width 0.6) (layer "F.Cu") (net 2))
 (segment (start 174.498 79.541266) (end 176.607734 81.651) (width 0.6) (layer "F.Cu") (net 2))
 (segment (start 176.607734 81.651) (end 179.249 81.651) (width 0.6) (layer "F.Cu") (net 2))
 (segment (start 178.75 63) (end 169 63) (width 0.6) (layer "F.Cu") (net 12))
 (segment (start 180.2125 68.25) (end 176.592782 68.25) (width 0.6) (layer "F.Cu") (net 9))
 (segment (start 191.095 68.853) (end 191.199 68.749) (width 0.6) (layer "F.Cu") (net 9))
 (segment (start 191.199 68.749) (end 198.369 68.749) (width 0.6) (layer "F.Cu") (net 9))
 (segment (start 179 73) (end 179 69.4625) (width 0.6) (layer "F.Cu") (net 9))
 (segment (start 175.599 67.256218) (end 175.599 65.901) (width 0.6) (layer "F.Cu") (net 9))
 (segment (start 180.599 64.651) (end 182.25 63) (width 0.6) (layer "F.Cu") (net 9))
 (segment (start 176.592782 68.25) (end 175.599 67.256218) (width 0.6) (layer "F.Cu") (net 9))
 (segment (start 188.392266 71.099) (end 191.095 73.801734) (width 0.6) (layer "F.Cu") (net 9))
 (segment (start 191.095 73.801734) (end 191.095 74.25) (width 0.6) (layer "F.Cu") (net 9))
 (segment (start 180.201 71.099) (end 188.392266 71.099) (width 0.6) (layer "F.Cu") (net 9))
 (segment (start 179 72.3) (end 180.201 71.099) (width 0.6) (layer "F.Cu") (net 9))
 (segment (start 191.095 74.25) (end 191.095 68.853) (width 0.6) (layer "F.Cu") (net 9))
 (segment (start 179 73) (end 179 72.3) (width 0.6) (layer "F.Cu") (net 9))
 (segment (start 198.369 68.749) (end 203.25 73.63) (width 0.6) (layer "F.Cu") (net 9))
 (segment (start 175.599 65.901) (end 176.849 64.651) (width 0.6) (layer "F.Cu") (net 9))
 (segment (start 176.849 64.651) (end 180.599 64.651) (width 0.6) (layer "F.Cu") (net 9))
 (segment (start 179 69.4625) (end 180.2125 68.25) (width 0.6) (layer "F.Cu") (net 9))
 (segment (start 191.095 74.25) (end 191.095 79.1625) (width 0.6) (layer "F.Cu") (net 9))
 (segment (start 179.792266 74.501) (end 180.5 73.793266) (width 0.6) (layer "F.Cu") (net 13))
 (segment (start 182 72.75) (end 182.25 72.5) (width 0.6) (layer "F.Cu") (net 13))
 (segment (start 174.25 65.5) (end 174.25 67.5) (width 0.6) (layer "F.Cu") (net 13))
 (segment (start 177 69.9) (end 177 73) (width 0.6) (layer "F.Cu") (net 13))
 (segment (start 176.65 69.9) (end 177 69.9) (width 0.6) (layer "F.Cu") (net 13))
 (segment (start 178.207734 74.501) (end 179.792266 74.501) (width 0.6) (layer "F.Cu") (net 13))
 (segment (start 168.5 65.5) (end 174.25 65.5) (width 0.6) (layer "F.Cu") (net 13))
 (segment (start 180.5 72.75) (end 182 72.75) (width 0.6) (layer "F.Cu") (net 13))
 (segment (start 177 73) (end 177 73.293266) (width 0.6) (layer "F.Cu") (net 13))
 (segment (start 182.25 72.5) (end 187.5 72.5) (width 0.6) (layer "F.Cu") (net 13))
 (segment (start 177 73.293266) (end 178.207734 74.501) (width 0.6) (layer "F.Cu") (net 13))
 (segment (start 174.25 67.5) (end 176.65 69.9) (width 0.6) (layer "F.Cu") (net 13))
 (segment (start 180.5 73.793266) (end 180.5 72.75) (width 0.6) (layer "F.Cu") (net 13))
 (segment (start 172.542782 67.5) (end 175.599 70.556218) (width 0.6) (layer "F.Cu") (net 10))
 (segment (start 175.599 70.556218) (end 175.599 77.849) (width 0.6) (layer "F.Cu") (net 10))
 (segment (start 177.5 78.25) (end 177.5 76) (width 0.6) (layer "F.Cu") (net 10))
 (segment (start 175.599 77.849) (end 176 78.25) (width 0.6) (layer "F.Cu") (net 10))
 (segment (start 177.6 76.1) (end 181.5 76.1) (width 0.6) (layer "F.Cu") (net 10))
 (segment (start 176 78.25) (end 177.5 78.25) (width 0.6) (layer "F.Cu") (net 10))
 (segment (start 168.5 67.5) (end 172.542782 67.5) (width 0.6) (layer "F.Cu") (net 10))
 (segment (start 177.5 76) (end 177.6 76.1) (width 0.6) (layer "F.Cu") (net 10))
 (segment (start 193.635 79.1625) (end 193.635 80.072098) (width 0.6) (layer "F.Cu") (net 7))
 (segment (start 193.635 80.072098) (end 194.983902 81.421) (width 0.6) (layer "F.Cu") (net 7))
 (segment (start 199.89805 81.421) (end 202.26705 83.79) (width 0.6) (layer "F.Cu") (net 7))
 (segment (start 194.983902 81.421) (end 199.89805 81.421) (width 0.6) (layer "F.Cu") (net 7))
 (segment (start 193.635 71.185) (end 193.635 79.1625) (width 0.6) (layer "F.Cu") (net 7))
 (segment (start 192.5 70.05) (end 193.635 71.185) (width 0.6) (layer "F.Cu") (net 7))
 (segment (start 193.635 79.1625) (end 193.635 78.252902) (width 0.6) (layer "F.Cu") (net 7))
 (segment (start 202.26705 83.79) (end 203.25 83.79) (width 0.6) (layer "F.Cu") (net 7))
 (segment (start 192.5375 67.2125) (end 192.5 67.25) (width 0.6) (layer "F.Cu") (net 1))
 (segment (start 192.5375 63.70625) (end 192.5375 67.2125) (width 0.6) (layer "F.Cu") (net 1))
 (segment (start 185.37 100.25) (end 181.42 100.25) (width 0.6) (layer "F.Cu") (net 11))
 (segment (start 201.1625 79.1625) (end 203.25 81.25) (width 0.6) (layer "F.Cu") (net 6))
 (segment (start 194.905 79.1625) (end 201.1625 79.1625) (width 0.6) (layer "F.Cu") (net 6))
 (segment (start 192.365 85.140853) (end 193.882853 83.623) (width 0.6) (layer "F.Cu") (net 4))
 (segment (start 193.882853 83.623) (end 198.003 83.623) (width 0.6) (layer "F.Cu") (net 4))
 (segment (start 192.365 86.3375) (end 192.365 85.140853) (width 0.6) (layer "F.Cu") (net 4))
 (segment (start 198.003 83.623) (end 203.25 88.87) (width 0.6) (layer "F.Cu") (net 4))
 (segment (start 187.5 78.5) (end 192.623 83.623) (width 0.6) (layer "F.Cu") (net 4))
 (segment (start 192.623 83.623) (end 193.882853 83.623) (width 0.6) (layer "F.Cu") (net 4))
 (segment (start 187.5 74.5) (end 187.5 78.5) (width 0.6) (layer "F.Cu") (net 4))
 (segment (start 192.365 79.1625) (end 192.365 80.359147) (width 0.6) (layer "F.Cu") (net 8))
 (segment (start 194.527853 82.522) (end 199.442 82.522) (width 0.6) (layer "F.Cu") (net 8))
 (segment (start 192.365 80.359147) (end 194.527853 82.522) (width 0.6) (layer "F.Cu") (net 8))
 (segment (start 199.442 82.522) (end 203.25 86.33) (width 0.6) (layer "F.Cu") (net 8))
 (segment (start 180.693782 78.149) (end 184.516902 78.149) (width 0.6) (layer "F.Cu") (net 5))
 (segment (start 194.338902 84.724) (end 196.564 84.724) (width 0.6) (layer "F.Cu") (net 5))
 (segment (start 196.564 84.724) (end 203.25 91.41) (width 0.6) (layer "F.Cu") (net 5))
 (segment (start 178.592782 80.25) (end 180.693782 78.149) (width 0.6) (layer "F.Cu") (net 5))
 (segment (start 184.516902 82.016902) (end 190.451 87.951) (width 0.6) (layer "F.Cu") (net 5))
 (segment (start 193.635 85.427902) (end 194.338902 84.724) (width 0.6) (layer "F.Cu") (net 5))
 (segment (start 193.635 86.3375) (end 193.635 85.427902) (width 0.6) (layer "F.Cu") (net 5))
 (segment (start 193.635 87.247098) (end 193.635 86.3375) (width 0.6) (layer "F.Cu") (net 5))
 (segment (start 190.451 87.951) (end 192.931098 87.951) (width 0.6) (layer "F.Cu") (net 5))
 (segment (start 184.516902 78.149) (end 184.516902 82.016902) (width 0.6) (layer "F.Cu") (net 5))
 (segment (start 177.5 80.25) (end 178.592782 80.25) (width 0.6) (layer "F.Cu") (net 5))
 (segment (start 192.931098 87.951) (end 193.635 87.247098) (width 0.6) (layer "F.Cu") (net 5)))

